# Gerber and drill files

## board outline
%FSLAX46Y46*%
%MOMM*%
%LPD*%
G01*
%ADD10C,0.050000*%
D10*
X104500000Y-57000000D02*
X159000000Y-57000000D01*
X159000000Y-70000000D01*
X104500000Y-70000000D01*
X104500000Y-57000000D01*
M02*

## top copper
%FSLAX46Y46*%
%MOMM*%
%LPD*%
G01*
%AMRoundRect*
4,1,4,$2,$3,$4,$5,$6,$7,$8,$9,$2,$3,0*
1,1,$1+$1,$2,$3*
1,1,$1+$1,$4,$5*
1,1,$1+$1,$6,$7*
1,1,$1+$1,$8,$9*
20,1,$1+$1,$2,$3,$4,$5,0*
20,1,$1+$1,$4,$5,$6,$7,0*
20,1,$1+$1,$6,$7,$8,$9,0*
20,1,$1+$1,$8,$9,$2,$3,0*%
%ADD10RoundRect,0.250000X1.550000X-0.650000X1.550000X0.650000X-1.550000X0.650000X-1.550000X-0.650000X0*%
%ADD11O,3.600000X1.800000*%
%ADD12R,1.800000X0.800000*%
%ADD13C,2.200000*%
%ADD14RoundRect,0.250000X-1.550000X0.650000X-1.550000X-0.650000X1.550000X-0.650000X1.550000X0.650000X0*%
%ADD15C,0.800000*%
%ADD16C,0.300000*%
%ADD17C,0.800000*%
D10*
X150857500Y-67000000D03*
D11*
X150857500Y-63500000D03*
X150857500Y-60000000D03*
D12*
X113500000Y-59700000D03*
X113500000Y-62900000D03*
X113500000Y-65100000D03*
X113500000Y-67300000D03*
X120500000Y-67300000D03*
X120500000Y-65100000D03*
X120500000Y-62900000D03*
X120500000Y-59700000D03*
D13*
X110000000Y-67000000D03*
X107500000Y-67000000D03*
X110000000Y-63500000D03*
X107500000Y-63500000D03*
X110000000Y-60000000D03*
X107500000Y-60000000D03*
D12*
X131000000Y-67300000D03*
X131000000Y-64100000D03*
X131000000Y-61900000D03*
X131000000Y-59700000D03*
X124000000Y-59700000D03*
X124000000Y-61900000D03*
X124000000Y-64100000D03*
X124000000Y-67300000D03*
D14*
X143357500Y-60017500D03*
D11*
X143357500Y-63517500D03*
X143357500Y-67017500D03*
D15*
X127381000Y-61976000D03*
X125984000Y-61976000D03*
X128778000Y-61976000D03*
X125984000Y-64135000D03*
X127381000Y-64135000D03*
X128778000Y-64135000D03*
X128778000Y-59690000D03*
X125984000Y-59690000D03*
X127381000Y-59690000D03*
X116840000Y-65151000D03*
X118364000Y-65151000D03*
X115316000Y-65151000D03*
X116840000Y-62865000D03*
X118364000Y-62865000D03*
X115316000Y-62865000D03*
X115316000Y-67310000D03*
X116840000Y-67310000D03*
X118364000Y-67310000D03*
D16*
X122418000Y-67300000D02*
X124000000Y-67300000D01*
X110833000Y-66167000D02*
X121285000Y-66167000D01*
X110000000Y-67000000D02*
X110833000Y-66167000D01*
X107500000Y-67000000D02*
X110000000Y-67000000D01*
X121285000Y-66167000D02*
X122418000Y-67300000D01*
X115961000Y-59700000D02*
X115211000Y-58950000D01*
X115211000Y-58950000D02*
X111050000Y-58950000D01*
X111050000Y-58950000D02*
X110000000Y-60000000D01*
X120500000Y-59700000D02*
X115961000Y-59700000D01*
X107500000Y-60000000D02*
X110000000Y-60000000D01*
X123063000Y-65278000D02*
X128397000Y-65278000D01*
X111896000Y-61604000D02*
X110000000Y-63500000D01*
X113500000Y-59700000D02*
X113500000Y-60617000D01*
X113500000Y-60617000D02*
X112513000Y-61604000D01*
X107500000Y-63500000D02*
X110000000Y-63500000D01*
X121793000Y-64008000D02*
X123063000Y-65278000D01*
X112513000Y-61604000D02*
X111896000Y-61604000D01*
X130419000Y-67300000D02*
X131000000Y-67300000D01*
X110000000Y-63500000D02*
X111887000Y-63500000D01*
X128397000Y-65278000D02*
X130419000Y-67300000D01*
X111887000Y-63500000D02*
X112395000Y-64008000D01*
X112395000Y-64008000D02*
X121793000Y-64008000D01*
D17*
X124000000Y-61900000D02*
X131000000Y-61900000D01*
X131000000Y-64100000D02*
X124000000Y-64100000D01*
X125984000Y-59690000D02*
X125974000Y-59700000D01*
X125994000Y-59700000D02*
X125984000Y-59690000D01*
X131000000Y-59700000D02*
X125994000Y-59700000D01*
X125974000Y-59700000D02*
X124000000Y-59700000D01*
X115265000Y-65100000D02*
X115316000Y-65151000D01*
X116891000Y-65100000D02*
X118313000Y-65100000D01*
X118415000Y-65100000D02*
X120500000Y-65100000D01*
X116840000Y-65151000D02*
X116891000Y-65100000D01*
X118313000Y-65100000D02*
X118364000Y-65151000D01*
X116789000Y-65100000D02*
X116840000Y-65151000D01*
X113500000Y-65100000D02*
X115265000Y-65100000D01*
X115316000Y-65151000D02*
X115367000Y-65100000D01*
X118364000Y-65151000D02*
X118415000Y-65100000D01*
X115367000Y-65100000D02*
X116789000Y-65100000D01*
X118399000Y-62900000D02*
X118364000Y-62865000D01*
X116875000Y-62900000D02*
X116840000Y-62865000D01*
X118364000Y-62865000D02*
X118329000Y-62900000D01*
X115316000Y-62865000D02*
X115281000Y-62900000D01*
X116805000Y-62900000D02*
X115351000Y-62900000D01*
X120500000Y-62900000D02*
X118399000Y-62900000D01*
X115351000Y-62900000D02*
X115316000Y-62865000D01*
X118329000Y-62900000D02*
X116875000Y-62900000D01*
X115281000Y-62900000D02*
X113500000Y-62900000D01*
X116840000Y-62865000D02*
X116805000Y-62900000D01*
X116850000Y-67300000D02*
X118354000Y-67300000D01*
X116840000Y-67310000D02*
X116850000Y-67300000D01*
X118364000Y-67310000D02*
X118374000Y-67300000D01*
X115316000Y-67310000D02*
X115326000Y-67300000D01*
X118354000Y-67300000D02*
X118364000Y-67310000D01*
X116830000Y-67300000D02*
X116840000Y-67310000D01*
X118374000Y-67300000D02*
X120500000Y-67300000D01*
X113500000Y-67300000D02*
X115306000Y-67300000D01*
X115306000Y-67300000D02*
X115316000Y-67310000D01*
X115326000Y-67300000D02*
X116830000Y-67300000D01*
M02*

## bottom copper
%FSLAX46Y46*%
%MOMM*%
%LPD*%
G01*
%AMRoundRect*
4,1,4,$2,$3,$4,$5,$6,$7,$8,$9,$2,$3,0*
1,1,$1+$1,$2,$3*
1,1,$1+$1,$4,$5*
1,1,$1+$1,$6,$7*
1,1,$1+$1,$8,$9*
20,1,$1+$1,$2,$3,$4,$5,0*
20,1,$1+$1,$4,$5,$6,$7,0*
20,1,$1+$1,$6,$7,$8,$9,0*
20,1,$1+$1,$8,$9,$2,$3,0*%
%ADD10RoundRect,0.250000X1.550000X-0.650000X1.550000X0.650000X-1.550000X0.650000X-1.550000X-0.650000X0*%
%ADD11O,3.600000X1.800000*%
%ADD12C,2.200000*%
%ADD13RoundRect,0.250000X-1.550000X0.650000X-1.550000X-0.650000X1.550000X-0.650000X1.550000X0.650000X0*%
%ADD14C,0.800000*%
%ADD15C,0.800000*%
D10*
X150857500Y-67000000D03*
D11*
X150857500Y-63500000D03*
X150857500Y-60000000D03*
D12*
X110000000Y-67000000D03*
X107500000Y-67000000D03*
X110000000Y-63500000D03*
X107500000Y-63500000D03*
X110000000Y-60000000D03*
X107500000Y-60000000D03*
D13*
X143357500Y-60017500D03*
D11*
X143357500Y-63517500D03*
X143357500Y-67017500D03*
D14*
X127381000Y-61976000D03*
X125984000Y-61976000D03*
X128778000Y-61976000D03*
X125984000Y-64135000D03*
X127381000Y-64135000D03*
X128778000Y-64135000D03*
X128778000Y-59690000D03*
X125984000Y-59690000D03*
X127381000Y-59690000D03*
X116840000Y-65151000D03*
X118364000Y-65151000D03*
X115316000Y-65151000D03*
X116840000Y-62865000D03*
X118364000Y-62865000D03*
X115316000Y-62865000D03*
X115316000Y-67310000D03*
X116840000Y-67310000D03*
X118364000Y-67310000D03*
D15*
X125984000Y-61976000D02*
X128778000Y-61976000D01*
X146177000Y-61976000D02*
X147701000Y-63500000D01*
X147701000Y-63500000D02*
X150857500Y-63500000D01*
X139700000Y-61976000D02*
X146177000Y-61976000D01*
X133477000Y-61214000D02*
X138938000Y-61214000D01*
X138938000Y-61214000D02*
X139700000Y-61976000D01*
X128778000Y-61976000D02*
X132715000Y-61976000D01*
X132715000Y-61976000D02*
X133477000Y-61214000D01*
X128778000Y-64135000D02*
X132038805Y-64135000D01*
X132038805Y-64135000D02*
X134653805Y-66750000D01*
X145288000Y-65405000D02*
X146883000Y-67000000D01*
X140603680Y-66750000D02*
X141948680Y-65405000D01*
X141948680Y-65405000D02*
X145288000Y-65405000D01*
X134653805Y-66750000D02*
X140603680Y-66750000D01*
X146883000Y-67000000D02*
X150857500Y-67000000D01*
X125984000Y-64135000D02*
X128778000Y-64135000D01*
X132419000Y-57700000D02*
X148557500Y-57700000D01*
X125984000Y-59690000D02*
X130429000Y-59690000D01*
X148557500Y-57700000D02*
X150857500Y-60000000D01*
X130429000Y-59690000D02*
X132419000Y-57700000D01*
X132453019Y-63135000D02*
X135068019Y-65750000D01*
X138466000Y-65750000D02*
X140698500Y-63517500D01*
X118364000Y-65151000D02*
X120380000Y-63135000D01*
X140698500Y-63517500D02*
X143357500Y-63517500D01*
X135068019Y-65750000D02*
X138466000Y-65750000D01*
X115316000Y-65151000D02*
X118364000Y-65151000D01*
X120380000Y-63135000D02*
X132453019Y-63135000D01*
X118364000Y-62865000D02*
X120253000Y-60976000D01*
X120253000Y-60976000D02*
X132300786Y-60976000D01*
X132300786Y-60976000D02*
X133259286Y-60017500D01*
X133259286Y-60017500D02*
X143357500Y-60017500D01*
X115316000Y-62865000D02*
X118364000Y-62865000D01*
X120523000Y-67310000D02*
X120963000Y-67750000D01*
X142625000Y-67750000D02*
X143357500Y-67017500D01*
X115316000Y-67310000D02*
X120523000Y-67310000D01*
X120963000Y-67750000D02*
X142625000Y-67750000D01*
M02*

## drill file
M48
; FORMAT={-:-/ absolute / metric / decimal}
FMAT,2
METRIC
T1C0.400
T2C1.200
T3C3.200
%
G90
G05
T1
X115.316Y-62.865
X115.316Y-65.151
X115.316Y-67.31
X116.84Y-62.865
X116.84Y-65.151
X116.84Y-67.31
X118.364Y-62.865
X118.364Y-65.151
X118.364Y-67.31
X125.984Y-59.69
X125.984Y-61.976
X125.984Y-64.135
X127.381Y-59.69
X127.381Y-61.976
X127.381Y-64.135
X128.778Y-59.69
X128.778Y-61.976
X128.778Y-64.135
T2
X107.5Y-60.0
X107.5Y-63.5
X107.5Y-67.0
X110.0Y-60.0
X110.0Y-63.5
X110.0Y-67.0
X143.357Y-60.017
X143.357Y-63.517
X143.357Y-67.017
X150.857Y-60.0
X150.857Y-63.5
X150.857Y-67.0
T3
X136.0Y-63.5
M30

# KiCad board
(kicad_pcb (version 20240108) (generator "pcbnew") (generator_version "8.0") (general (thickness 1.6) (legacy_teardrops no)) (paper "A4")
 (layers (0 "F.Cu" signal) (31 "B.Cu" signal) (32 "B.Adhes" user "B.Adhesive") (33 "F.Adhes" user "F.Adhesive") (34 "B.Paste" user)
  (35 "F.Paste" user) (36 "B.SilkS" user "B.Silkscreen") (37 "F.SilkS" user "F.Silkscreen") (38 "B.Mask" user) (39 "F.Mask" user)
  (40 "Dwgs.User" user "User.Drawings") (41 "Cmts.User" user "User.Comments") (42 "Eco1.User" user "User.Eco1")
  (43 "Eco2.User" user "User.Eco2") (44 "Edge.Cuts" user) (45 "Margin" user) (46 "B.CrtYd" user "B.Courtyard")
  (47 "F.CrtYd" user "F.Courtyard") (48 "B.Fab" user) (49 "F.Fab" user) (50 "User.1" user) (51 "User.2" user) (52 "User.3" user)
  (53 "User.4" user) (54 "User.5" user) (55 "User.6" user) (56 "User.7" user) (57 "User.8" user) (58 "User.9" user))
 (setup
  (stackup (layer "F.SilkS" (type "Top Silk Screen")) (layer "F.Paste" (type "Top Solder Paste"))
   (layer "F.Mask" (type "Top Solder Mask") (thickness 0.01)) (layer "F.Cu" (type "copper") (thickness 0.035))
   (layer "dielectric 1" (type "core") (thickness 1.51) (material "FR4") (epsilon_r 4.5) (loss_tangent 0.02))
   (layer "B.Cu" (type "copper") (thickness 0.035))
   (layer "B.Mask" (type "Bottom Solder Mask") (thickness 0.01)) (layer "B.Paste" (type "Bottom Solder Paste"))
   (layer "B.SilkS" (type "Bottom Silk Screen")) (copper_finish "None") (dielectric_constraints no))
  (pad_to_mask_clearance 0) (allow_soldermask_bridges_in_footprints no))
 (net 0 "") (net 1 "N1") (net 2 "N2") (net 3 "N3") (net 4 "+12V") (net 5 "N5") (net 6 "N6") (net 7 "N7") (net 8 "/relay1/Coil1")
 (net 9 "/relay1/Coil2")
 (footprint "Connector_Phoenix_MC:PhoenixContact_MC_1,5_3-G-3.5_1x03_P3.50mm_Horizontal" (layer "F.Cu") (at 150.8575 67 90)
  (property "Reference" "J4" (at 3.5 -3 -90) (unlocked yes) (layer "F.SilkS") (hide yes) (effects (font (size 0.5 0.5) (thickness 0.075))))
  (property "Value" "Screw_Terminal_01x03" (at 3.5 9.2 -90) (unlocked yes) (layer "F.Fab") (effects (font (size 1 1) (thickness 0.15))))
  (pad "1" thru_hole roundrect (at 0 0 90) (size 1.8 3.6) (drill 1.2) (layers "*.Cu" "*.Mask") (remove_unused_layers no)
   (roundrect_rratio 0.138889) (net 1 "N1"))
  (pad "2" thru_hole oval (at 3.5 0 90) (size 1.8 3.6) (drill 1.2) (layers "*.Cu" "*.Mask") (remove_unused_layers no) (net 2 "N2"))
  (pad "3" thru_hole oval (at 7 0 90) (size 1.8 3.6) (drill 1.2) (layers "*.Cu" "*.Mask") (remove_unused_layers no) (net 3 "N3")))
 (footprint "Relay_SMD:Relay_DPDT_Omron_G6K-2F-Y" (layer "F.Cu") (at 117 63.5)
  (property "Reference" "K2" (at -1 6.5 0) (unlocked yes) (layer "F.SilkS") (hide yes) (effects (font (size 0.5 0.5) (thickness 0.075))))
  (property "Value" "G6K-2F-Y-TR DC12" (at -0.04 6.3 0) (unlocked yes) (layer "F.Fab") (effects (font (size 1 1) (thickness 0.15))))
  (pad "1" smd rect (at -3.5 -3.8) (size 1.8 0.8) (layers "F.Cu" "F.Paste" "F.Mask") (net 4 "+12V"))
  (pad "2" smd rect (at -3.5 -0.6) (size 1.8 0.8) (layers "F.Cu" "F.Paste" "F.Mask") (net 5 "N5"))
  (pad "3" smd rect (at -3.5 1.6) (size 1.8 0.8) (layers "F.Cu" "F.Paste" "F.Mask") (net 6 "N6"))
  (pad "4" smd rect (at -3.5 3.8) (size 1.8 0.8) (layers "F.Cu" "F.Paste" "F.Mask") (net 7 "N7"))
  (pad "5" smd rect (at 3.5 3.8) (size 1.8 0.8) (layers "F.Cu" "F.Paste" "F.Mask") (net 7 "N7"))
  (pad "6" smd rect (at 3.5 1.6) (size 1.8 0.8) (layers "F.Cu" "F.Paste" "F.Mask") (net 6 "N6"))
  (pad "7" smd rect (at 3.5 -0.6) (size 1.8 0.8) (layers "F.Cu" "F.Paste" "F.Mask") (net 5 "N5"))
  (pad "8" smd rect (at 3.5 -3.8) (size 1.8 0.8) (layers "F.Cu" "F.Paste" "F.Mask") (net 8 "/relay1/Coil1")))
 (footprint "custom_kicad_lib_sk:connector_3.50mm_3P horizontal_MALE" (layer "F.Cu") (at 110 63.5 -90)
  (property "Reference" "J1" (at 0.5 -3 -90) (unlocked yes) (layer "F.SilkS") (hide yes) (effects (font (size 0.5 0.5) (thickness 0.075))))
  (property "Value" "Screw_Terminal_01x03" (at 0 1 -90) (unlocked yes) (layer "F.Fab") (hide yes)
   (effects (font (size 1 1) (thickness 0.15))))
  (pad "1" thru_hole circle (at 3.5 0 270) (size 2.2 2.2) (drill 1.2) (layers "*.Cu" "*.Mask") (remove_unused_layers no)
   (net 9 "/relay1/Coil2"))
  (pad "1" thru_hole circle (at 3.5 2.5 270) (size 2.2 2.2) (drill 1.2) (layers "*.Cu" "*.Mask") (remove_unused_layers no)
   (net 9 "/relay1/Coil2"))
  (pad "2" thru_hole circle (at 0 0 270) (size 2.2 2.2) (drill 1.2) (layers "*.Cu" "*.Mask") (remove_unused_layers no) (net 4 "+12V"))
  (pad "2" thru_hole circle (at 0 2.5 270) (size 2.2 2.2) (drill 1.2) (layers "*.Cu" "*.Mask") (remove_unused_layers no) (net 4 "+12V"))
  (pad "3" thru_hole circle (at -3.5 0 270) (size 2.2 2.2) (drill 1.2) (layers "*.Cu" "*.Mask") (remove_unused_layers no)
   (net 8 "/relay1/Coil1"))
  (pad "3" thru_hole circle (at -3.5 2.5 270) (size 2.2 2.2) (drill 1.2) (layers "*.Cu" "*.Mask") (remove_unused_layers no)
   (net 8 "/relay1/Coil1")))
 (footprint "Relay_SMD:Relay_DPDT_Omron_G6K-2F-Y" (layer "F.Cu") (at 127.5 63.5 180)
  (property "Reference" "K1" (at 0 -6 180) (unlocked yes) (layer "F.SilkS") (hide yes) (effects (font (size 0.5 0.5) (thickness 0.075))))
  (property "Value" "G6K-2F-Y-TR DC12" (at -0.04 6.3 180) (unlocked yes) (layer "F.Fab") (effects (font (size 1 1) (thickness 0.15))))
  (pad "1" smd rect (at -3.5 -3.8 180) (size 1.8 0.8) (layers "F.Cu" "F.Paste" "F.Mask") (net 4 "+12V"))
  (pad "2" smd rect (at -3.5 -0.6 180) (size 1.8 0.8) (layers "F.Cu" "F.Paste" "F.Mask") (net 1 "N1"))
  (pad "3" smd rect (at -3.5 1.6 180) (size 1.8 0.8) (layers "F.Cu" "F.Paste" "F.Mask") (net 2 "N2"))
  (pad "4" smd rect (at -3.5 3.8 180) (size 1.8 0.8) (layers "F.Cu" "F.Paste" "F.Mask") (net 3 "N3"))
  (pad "5" smd rect (at 3.5 3.8 180) (size 1.8 0.8) (layers "F.Cu" "F.Paste" "F.Mask") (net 3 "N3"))
  (pad "6" smd rect (at 3.5 1.6 180) (size 1.8 0.8) (layers "F.Cu" "F.Paste" "F.Mask") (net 2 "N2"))
  (pad "7" smd rect (at 3.5 -0.6 180) (size 1.8 0.8) (layers "F.Cu" "F.Paste" "F.Mask") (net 1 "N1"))
  (pad "8" smd rect (at 3.5 -3.8 180) (size 1.8 0.8) (layers "F.Cu" "F.Paste" "F.Mask") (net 9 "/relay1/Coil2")))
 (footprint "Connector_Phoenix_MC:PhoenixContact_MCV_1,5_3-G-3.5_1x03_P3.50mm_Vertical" (layer "F.Cu") (at 143.3575 60.0175 -90)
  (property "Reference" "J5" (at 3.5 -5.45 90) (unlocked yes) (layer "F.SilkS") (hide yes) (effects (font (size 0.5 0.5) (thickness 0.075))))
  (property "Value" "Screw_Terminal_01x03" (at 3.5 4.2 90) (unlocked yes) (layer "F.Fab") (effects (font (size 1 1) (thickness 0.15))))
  (pad "1" thru_hole roundrect (at 0 0 270) (size 1.8 3.6) (drill 1.2) (layers "*.Cu" "*.Mask") (remove_unused_layers no)
   (roundrect_rratio 0.138889) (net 5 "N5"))
  (pad "2" thru_hole oval (at 3.5 0 270) (size 1.8 3.6) (drill 1.2) (layers "*.Cu" "*.Mask") (remove_unused_layers no) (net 6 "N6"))
  (pad "3" thru_hole oval (at 7 0 270) (size 1.8 3.6) (drill 1.2) (layers "*.Cu" "*.Mask") (remove_unused_layers no) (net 7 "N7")))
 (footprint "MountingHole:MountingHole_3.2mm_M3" (layer "F.Cu") (at 136 63.5)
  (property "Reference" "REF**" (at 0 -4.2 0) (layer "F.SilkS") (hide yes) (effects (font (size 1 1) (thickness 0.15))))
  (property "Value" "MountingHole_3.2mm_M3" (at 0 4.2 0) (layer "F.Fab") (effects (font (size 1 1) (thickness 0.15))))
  (pad "" np_thru_hole circle (at 0 0) (size 3.2 3.2) (drill 3.2) (layers "*.Cu" "*.Mask")))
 (gr_rect (start 104.5 57) (end 159 70) (stroke (width 0.05) (type default)) (fill none) (layer "Edge.Cuts"))
 (segment (start 122.418 67.3) (end 124 67.3) (width 0.3) (layer "F.Cu") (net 9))
 (segment (start 110.833 66.167) (end 121.285 66.167) (width 0.3) (layer "F.Cu") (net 9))
 (segment (start 110 67) (end 110.833 66.167) (width 0.3) (layer "F.Cu") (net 9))
 (segment (start 107.5 67) (end 110 67) (width 0.3) (layer "F.Cu") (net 9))
 (segment (start 121.285 66.167) (end 122.418 67.3) (width 0.3) (layer "F.Cu") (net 9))
 (segment (start 115.961 59.7) (end 115.211 58.95) (width 0.3) (layer "F.Cu") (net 8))
 (segment (start 115.211 58.95) (end 111.05 58.95) (width 0.3) (layer "F.Cu") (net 8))
 (segment (start 111.05 58.95) (end 110 60) (width 0.3) (layer "F.Cu") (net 8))
 (segment (start 120.5 59.7) (end 115.961 59.7) (width 0.3) (layer "F.Cu") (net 8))
 (segment (start 107.5 60) (end 110 60) (width 0.3) (layer "F.Cu") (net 8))
 (segment (start 123.063 65.278) (end 128.397 65.278) (width 0.3) (layer "F.Cu") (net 4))
 (segment (start 111.896 61.604) (end 110 63.5) (width 0.3) (layer "F.Cu") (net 4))
 (segment (start 113.5 59.7) (end 113.5 60.617) (width 0.3) (layer "F.Cu") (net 4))
 (segment (start 113.5 60.617) (end 112.513 61.604) (width 0.3) (layer "F.Cu") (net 4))
 (segment (start 107.5 63.5) (end 110 63.5) (width 0.3) (layer "F.Cu") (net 4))
 (segment (start 121.793 64.008) (end 123.063 65.278) (width 0.3) (layer "F.Cu") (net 4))
 (segment (start 112.513 61.604) (end 111.896 61.604) (width 0.3) (layer "F.Cu") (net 4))
 (segment (start 130.419 67.3) (end 131 67.3) (width 0.3) (layer "F.Cu") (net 4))
 (segment (start 110 63.5) (end 111.887 63.5) (width 0.3) (layer "F.Cu") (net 4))
 (segment (start 128.397 65.278) (end 130.419 67.3) (width 0.3) (layer "F.Cu") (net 4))
 (segment (start 111.887 63.5) (end 112.395 64.008) (width 0.3) (layer "F.Cu") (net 4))
 (segment (start 112.395 64.008) (end 121.793 64.008) (width 0.3) (layer "F.Cu") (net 4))
 (segment (start 124 61.9) (end 131 61.9) (width 0.8) (layer "F.Cu") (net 2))
 (via (at 127.381 61.976) (size 0.8) (drill 0.4) (layers "F.Cu" "B.Cu") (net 2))
 (via (at 125.984 61.976) (size 0.8) (drill 0.4) (layers "F.Cu" "B.Cu") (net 2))
 (via (at 128.778 61.976) (size 0.8) (drill 0.4) (layers "F.Cu" "B.Cu") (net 2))
 (segment (start 125.984 61.976) (end 128.778 61.976) (width 0.8) (layer "B.Cu") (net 2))
 (segment (start 146.177 61.976) (end 147.701 63.5) (width 0.8) (layer "B.Cu") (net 2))
 (segment (start 147.701 63.5) (end 150.8575 63.5) (width 0.8) (layer "B.Cu") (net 2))
 (segment (start 139.7 61.976) (end 146.177 61.976) (width 0.8) (layer "B.Cu") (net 2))
 (segment (start 133.477 61.214) (end 138.938 61.214) (width 0.8) (layer "B.Cu") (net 2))
 (segment (start 138.938 61.214) (end 139.7 61.976) (width 0.8) (layer "B.Cu") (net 2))
 (segment (start 128.778 61.976) (end 132.715 61.976) (width 0.8) (layer "B.Cu") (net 2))
 (segment (start 132.715 61.976) (end 133.477 61.214) (width 0.8) (layer "B.Cu") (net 2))
 (segment (start 131 64.1) (end 124 64.1) (width 0.8) (layer "F.Cu") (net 1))
 (via (at 125.984 64.135) (size 0.8) (drill 0.4) (layers "F.Cu" "B.Cu") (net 1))
 (via (at 127.381 64.135) (size 0.8) (drill 0.4) (layers "F.Cu" "B.Cu") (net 1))
 (via (at 128.778 64.135) (size 0.8) (drill 0.4) (layers "F.Cu" "B.Cu") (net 1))
 (segment (start 128.778 64.135) (end 132.038805 64.135) (width 0.8) (layer "B.Cu") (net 1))
 (segment (start 132.038805 64.135) (end 134.653805 66.75) (width 0.8) (layer "B.Cu") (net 1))
 (segment (start 145.288 65.405) (end 146.883 67) (width 0.8) (layer "B.Cu") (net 1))
 (segment (start 140.60368 66.75) (end 141.94868 65.405) (width 0.8) (layer "B.Cu") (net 1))
 (segment (start 141.94868 65.405) (end 145.288 65.405) (width 0.8) (layer "B.Cu") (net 1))
 (segment (start 134.653805 66.75) (end 140.60368 66.75) (width 0.8) (layer "B.Cu") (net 1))
 (segment (start 146.883 67) (end 150.8575 67) (width 0.8) (layer "B.Cu") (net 1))
 (segment (start 125.984 64.135) (end 128.778 64.135) (width 0.8) (layer "B.Cu") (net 1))
 (segment (start 125.984 59.69) (end 125.974 59.7) (width 0.8) (layer "F.Cu") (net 3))
 (segment (start 125.994 59.7) (end 125.984 59.69) (width 0.8) (layer "F.Cu") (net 3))
 (segment (start 131 59.7) (end 125.994 59.7) (width 0.8) (layer "F.Cu") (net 3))
 (segment (start 125.974 59.7) (end 124 59.7) (width 0.8) (layer "F.Cu") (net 3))
 (via (at 128.778 59.69) (size 0.8) (drill 0.4) (layers "F.Cu" "B.Cu") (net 3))
 (via (at 125.984 59.69) (size 0.8) (drill 0.4) (layers "F.Cu" "B.Cu") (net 3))
 (via (at 127.381 59.69) (size 0.8) (drill 0.4) (layers "F.Cu" "B.Cu") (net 3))
 (segment (start 132.419 57.7) (end 148.5575 57.7) (width 0.8) (layer "B.Cu") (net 3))
 (segment (start 125.984 59.69) (end 130.429 59.69) (width 0.8) (layer "B.Cu") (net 3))
 (segment (start 148.5575 57.7) (end 150.8575 60) (width 0.8) (layer "B.Cu") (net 3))
 (segment (start 130.429 59.69) (end 132.419 57.7) (width 0.8) (layer "B.Cu") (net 3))
 (segment (start 115.265 65.1) (end 115.316 65.151) (width 0.8) (layer "F.Cu") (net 6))
 (segment (start 116.891 65.1) (end 118.313 65.1) (width 0.8) (layer "F.Cu") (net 6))
 (segment (start 118.415 65.1) (end 120.5 65.1) (width 0.8) (layer "F.Cu") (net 6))
 (segment (start 116.84 65.151) (end 116.891 65.1) (width 0.8) (layer "F.Cu") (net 6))
 (segment (start 118.313 65.1) (end 118.364 65.151) (width 0.8) (layer "F.Cu") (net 6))
 (segment (start 116.789 65.1) (end 116.84 65.151) (width 0.8) (layer "F.Cu") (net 6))
 (segment (start 113.5 65.1) (end 115.265 65.1) (width 0.8) (layer "F.Cu") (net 6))
 (segment (start 115.316 65.151) (end 115.367 65.1) (width 0.8) (layer "F.Cu") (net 6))
 (segment (start 118.364 65.151) (end 118.415 65.1) (width 0.8) (layer "F.Cu") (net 6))
 (segment (start 115.367 65.1) (end 116.789 65.1) (width 0.8) (layer "F.Cu") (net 6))
 (via (at 116.84 65.151) (size 0.8) (drill 0.4) (layers "F.Cu" "B.Cu") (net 6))
 (via (at 118.364 65.151) (size 0.8) (drill 0.4) (layers "F.Cu" "B.Cu") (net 6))
 (via (at 115.316 65.151) (size 0.8) (drill 0.4) (layers "F.Cu" "B.Cu") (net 6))
 (segment (start 132.453019 63.135) (end 135.068019 65.75) (width 0.8) (layer "B.Cu") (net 6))
 (segment (start 138.466 65.75) (end 140.6985 63.5175) (width 0.8) (layer "B.Cu") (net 6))
 (segment (start 118.364 65.151) (end 120.38 63.135) (width 0.8) (layer "B.Cu") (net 6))
 (segment (start 140.6985 63.5175) (end 143.3575 63.5175) (width 0.8) (layer "B.Cu") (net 6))
 (segment (start 135.068019 65.75) (end 138.466 65.75) (width 0.8) (layer "B.Cu") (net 6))
 (segment (start 115.316 65.151) (end 118.364 65.151) (width 0.8) (layer "B.Cu") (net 6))
 (segment (start 120.38 63.135) (end 132.453019 63.135) (width 0.8) (layer "B.Cu") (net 6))
 (segment (start 118.399 62.9) (end 118.364 62.865) (width 0.8) (layer "F.Cu") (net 5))
 (segment (start 116.875 62.9) (end 116.84 62.865) (width 0.8) (layer "F.Cu") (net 5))
 (segment (start 118.364 62.865) (end 118.329 62.9) (width 0.8) (layer "F.Cu") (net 5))
 (segment (start 115.316 62.865) (end 115.281 62.9) (width 0.8) (layer "F.Cu") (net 5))
 (segment (start 116.805 62.9) (end 115.351 62.9) (width 0.8) (layer "F.Cu") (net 5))
 (segment (start 120.5 62.9) (end 118.399 62.9) (width 0.8) (layer "F.Cu") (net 5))
 (segment (start 115.351 62.9) (end 115.316 62.865) (width 0.8) (layer "F.Cu") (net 5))
 (segment (start 118.329 62.9) (end 116.875 62.9) (width 0.8) (layer "F.Cu") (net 5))
 (segment (start 115.281 62.9) (end 113.5 62.9) (width 0.8) (layer "F.Cu") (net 5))
 (segment (start 116.84 62.865) (end 116.805 62.9) (width 0.8) (layer "F.Cu") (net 5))
 (via (at 116.84 62.865) (size 0.8) (drill 0.4) (layers "F.Cu" "B.Cu") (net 5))
 (via (at 118.364 62.865) (size 0.8) (drill 0.4) (layers "F.Cu" "B.Cu") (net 5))
 (via (at 115.316 62.865) (size 0.8) (drill 0.4) (layers "F.Cu" "B.Cu") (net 5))
 (segment (start 118.364 62.865) (end 120.253 60.976) (width 0.8) (layer "B.Cu") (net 5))
 (segment (start 120.253 60.976) (end 132.300786 60.976) (width 0.8) (layer "B.Cu") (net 5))
 (segment (start 132.300786 60.976) (end 133.259286 60.0175) (width 0.8) (layer "B.Cu") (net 5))
 (segment (start 133.259286 60.0175) (end 143.3575 60.0175) (width 0.8) (layer "B.Cu") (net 5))
 (segment (start 115.316 62.865) (end 118.364 62.865) (width 0.8) (layer "B.Cu") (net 5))
 (segment (start 116.85 67.3) (end 118.354 67.3) (width 0.8) (layer "F.Cu") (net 7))
 (segment (start 116.84 67.31) (end 116.85 67.3) (width 0.8) (layer "F.Cu") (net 7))
 (segment (start 118.364 67.31) (end 118.374 67.3) (width 0.8) (layer "F.Cu") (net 7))
 (segment (start 115.316 67.31) (end 115.326 67.3) (width 0.8) (layer "F.Cu") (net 7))
 (segment (start 118.354 67.3) (end 118.364 67.31) (width 0.8) (layer "F.Cu") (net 7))
 (segment (start 116.83 67.3) (end 116.84 67.31) (width 0.8) (layer "F.Cu") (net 7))
 (segment (start 118.374 67.3) (end 120.5 67.3) (width 0.8) (layer "F.Cu") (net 7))
 (segment (start 113.5 67.3) (end 115.306 67.3) (width 0.8) (layer "F.Cu") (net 7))
 (segment (start 115.306 67.3) (end 115.316 67.31) (width 0.8) (layer "F.Cu") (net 7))
 (segment (start 115.326 67.3) (end 116.83 67.3) (width 0.8) (layer "F.Cu") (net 7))
 (via (at 115.316 67.31) (size 0.8) (drill 0.4) (layers "F.Cu" "B.Cu") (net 7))
 (via (at 116.84 67.31) (size 0.8) (drill 0.4) (layers "F.Cu" "B.Cu") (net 7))
 (via (at 118.364 67.31) (size 0.8) (drill 0.4) (layers "F.Cu" "B.Cu") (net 7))
 (segment (start 120.523 67.31) (end 120.963 67.75) (width 0.8) (layer "B.Cu") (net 7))
 (segment (start 142.625 67.75) (end 143.3575 67.0175) (width 0.8) (layer "B.Cu") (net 7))
 (segment (start 115.316 67.31) (end 120.523 67.31) (width 0.8) (layer "B.Cu") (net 7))
 (segment (start 120.963 67.75) (end 142.625 67.75) (width 0.8) (layer "B.Cu") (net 7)))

